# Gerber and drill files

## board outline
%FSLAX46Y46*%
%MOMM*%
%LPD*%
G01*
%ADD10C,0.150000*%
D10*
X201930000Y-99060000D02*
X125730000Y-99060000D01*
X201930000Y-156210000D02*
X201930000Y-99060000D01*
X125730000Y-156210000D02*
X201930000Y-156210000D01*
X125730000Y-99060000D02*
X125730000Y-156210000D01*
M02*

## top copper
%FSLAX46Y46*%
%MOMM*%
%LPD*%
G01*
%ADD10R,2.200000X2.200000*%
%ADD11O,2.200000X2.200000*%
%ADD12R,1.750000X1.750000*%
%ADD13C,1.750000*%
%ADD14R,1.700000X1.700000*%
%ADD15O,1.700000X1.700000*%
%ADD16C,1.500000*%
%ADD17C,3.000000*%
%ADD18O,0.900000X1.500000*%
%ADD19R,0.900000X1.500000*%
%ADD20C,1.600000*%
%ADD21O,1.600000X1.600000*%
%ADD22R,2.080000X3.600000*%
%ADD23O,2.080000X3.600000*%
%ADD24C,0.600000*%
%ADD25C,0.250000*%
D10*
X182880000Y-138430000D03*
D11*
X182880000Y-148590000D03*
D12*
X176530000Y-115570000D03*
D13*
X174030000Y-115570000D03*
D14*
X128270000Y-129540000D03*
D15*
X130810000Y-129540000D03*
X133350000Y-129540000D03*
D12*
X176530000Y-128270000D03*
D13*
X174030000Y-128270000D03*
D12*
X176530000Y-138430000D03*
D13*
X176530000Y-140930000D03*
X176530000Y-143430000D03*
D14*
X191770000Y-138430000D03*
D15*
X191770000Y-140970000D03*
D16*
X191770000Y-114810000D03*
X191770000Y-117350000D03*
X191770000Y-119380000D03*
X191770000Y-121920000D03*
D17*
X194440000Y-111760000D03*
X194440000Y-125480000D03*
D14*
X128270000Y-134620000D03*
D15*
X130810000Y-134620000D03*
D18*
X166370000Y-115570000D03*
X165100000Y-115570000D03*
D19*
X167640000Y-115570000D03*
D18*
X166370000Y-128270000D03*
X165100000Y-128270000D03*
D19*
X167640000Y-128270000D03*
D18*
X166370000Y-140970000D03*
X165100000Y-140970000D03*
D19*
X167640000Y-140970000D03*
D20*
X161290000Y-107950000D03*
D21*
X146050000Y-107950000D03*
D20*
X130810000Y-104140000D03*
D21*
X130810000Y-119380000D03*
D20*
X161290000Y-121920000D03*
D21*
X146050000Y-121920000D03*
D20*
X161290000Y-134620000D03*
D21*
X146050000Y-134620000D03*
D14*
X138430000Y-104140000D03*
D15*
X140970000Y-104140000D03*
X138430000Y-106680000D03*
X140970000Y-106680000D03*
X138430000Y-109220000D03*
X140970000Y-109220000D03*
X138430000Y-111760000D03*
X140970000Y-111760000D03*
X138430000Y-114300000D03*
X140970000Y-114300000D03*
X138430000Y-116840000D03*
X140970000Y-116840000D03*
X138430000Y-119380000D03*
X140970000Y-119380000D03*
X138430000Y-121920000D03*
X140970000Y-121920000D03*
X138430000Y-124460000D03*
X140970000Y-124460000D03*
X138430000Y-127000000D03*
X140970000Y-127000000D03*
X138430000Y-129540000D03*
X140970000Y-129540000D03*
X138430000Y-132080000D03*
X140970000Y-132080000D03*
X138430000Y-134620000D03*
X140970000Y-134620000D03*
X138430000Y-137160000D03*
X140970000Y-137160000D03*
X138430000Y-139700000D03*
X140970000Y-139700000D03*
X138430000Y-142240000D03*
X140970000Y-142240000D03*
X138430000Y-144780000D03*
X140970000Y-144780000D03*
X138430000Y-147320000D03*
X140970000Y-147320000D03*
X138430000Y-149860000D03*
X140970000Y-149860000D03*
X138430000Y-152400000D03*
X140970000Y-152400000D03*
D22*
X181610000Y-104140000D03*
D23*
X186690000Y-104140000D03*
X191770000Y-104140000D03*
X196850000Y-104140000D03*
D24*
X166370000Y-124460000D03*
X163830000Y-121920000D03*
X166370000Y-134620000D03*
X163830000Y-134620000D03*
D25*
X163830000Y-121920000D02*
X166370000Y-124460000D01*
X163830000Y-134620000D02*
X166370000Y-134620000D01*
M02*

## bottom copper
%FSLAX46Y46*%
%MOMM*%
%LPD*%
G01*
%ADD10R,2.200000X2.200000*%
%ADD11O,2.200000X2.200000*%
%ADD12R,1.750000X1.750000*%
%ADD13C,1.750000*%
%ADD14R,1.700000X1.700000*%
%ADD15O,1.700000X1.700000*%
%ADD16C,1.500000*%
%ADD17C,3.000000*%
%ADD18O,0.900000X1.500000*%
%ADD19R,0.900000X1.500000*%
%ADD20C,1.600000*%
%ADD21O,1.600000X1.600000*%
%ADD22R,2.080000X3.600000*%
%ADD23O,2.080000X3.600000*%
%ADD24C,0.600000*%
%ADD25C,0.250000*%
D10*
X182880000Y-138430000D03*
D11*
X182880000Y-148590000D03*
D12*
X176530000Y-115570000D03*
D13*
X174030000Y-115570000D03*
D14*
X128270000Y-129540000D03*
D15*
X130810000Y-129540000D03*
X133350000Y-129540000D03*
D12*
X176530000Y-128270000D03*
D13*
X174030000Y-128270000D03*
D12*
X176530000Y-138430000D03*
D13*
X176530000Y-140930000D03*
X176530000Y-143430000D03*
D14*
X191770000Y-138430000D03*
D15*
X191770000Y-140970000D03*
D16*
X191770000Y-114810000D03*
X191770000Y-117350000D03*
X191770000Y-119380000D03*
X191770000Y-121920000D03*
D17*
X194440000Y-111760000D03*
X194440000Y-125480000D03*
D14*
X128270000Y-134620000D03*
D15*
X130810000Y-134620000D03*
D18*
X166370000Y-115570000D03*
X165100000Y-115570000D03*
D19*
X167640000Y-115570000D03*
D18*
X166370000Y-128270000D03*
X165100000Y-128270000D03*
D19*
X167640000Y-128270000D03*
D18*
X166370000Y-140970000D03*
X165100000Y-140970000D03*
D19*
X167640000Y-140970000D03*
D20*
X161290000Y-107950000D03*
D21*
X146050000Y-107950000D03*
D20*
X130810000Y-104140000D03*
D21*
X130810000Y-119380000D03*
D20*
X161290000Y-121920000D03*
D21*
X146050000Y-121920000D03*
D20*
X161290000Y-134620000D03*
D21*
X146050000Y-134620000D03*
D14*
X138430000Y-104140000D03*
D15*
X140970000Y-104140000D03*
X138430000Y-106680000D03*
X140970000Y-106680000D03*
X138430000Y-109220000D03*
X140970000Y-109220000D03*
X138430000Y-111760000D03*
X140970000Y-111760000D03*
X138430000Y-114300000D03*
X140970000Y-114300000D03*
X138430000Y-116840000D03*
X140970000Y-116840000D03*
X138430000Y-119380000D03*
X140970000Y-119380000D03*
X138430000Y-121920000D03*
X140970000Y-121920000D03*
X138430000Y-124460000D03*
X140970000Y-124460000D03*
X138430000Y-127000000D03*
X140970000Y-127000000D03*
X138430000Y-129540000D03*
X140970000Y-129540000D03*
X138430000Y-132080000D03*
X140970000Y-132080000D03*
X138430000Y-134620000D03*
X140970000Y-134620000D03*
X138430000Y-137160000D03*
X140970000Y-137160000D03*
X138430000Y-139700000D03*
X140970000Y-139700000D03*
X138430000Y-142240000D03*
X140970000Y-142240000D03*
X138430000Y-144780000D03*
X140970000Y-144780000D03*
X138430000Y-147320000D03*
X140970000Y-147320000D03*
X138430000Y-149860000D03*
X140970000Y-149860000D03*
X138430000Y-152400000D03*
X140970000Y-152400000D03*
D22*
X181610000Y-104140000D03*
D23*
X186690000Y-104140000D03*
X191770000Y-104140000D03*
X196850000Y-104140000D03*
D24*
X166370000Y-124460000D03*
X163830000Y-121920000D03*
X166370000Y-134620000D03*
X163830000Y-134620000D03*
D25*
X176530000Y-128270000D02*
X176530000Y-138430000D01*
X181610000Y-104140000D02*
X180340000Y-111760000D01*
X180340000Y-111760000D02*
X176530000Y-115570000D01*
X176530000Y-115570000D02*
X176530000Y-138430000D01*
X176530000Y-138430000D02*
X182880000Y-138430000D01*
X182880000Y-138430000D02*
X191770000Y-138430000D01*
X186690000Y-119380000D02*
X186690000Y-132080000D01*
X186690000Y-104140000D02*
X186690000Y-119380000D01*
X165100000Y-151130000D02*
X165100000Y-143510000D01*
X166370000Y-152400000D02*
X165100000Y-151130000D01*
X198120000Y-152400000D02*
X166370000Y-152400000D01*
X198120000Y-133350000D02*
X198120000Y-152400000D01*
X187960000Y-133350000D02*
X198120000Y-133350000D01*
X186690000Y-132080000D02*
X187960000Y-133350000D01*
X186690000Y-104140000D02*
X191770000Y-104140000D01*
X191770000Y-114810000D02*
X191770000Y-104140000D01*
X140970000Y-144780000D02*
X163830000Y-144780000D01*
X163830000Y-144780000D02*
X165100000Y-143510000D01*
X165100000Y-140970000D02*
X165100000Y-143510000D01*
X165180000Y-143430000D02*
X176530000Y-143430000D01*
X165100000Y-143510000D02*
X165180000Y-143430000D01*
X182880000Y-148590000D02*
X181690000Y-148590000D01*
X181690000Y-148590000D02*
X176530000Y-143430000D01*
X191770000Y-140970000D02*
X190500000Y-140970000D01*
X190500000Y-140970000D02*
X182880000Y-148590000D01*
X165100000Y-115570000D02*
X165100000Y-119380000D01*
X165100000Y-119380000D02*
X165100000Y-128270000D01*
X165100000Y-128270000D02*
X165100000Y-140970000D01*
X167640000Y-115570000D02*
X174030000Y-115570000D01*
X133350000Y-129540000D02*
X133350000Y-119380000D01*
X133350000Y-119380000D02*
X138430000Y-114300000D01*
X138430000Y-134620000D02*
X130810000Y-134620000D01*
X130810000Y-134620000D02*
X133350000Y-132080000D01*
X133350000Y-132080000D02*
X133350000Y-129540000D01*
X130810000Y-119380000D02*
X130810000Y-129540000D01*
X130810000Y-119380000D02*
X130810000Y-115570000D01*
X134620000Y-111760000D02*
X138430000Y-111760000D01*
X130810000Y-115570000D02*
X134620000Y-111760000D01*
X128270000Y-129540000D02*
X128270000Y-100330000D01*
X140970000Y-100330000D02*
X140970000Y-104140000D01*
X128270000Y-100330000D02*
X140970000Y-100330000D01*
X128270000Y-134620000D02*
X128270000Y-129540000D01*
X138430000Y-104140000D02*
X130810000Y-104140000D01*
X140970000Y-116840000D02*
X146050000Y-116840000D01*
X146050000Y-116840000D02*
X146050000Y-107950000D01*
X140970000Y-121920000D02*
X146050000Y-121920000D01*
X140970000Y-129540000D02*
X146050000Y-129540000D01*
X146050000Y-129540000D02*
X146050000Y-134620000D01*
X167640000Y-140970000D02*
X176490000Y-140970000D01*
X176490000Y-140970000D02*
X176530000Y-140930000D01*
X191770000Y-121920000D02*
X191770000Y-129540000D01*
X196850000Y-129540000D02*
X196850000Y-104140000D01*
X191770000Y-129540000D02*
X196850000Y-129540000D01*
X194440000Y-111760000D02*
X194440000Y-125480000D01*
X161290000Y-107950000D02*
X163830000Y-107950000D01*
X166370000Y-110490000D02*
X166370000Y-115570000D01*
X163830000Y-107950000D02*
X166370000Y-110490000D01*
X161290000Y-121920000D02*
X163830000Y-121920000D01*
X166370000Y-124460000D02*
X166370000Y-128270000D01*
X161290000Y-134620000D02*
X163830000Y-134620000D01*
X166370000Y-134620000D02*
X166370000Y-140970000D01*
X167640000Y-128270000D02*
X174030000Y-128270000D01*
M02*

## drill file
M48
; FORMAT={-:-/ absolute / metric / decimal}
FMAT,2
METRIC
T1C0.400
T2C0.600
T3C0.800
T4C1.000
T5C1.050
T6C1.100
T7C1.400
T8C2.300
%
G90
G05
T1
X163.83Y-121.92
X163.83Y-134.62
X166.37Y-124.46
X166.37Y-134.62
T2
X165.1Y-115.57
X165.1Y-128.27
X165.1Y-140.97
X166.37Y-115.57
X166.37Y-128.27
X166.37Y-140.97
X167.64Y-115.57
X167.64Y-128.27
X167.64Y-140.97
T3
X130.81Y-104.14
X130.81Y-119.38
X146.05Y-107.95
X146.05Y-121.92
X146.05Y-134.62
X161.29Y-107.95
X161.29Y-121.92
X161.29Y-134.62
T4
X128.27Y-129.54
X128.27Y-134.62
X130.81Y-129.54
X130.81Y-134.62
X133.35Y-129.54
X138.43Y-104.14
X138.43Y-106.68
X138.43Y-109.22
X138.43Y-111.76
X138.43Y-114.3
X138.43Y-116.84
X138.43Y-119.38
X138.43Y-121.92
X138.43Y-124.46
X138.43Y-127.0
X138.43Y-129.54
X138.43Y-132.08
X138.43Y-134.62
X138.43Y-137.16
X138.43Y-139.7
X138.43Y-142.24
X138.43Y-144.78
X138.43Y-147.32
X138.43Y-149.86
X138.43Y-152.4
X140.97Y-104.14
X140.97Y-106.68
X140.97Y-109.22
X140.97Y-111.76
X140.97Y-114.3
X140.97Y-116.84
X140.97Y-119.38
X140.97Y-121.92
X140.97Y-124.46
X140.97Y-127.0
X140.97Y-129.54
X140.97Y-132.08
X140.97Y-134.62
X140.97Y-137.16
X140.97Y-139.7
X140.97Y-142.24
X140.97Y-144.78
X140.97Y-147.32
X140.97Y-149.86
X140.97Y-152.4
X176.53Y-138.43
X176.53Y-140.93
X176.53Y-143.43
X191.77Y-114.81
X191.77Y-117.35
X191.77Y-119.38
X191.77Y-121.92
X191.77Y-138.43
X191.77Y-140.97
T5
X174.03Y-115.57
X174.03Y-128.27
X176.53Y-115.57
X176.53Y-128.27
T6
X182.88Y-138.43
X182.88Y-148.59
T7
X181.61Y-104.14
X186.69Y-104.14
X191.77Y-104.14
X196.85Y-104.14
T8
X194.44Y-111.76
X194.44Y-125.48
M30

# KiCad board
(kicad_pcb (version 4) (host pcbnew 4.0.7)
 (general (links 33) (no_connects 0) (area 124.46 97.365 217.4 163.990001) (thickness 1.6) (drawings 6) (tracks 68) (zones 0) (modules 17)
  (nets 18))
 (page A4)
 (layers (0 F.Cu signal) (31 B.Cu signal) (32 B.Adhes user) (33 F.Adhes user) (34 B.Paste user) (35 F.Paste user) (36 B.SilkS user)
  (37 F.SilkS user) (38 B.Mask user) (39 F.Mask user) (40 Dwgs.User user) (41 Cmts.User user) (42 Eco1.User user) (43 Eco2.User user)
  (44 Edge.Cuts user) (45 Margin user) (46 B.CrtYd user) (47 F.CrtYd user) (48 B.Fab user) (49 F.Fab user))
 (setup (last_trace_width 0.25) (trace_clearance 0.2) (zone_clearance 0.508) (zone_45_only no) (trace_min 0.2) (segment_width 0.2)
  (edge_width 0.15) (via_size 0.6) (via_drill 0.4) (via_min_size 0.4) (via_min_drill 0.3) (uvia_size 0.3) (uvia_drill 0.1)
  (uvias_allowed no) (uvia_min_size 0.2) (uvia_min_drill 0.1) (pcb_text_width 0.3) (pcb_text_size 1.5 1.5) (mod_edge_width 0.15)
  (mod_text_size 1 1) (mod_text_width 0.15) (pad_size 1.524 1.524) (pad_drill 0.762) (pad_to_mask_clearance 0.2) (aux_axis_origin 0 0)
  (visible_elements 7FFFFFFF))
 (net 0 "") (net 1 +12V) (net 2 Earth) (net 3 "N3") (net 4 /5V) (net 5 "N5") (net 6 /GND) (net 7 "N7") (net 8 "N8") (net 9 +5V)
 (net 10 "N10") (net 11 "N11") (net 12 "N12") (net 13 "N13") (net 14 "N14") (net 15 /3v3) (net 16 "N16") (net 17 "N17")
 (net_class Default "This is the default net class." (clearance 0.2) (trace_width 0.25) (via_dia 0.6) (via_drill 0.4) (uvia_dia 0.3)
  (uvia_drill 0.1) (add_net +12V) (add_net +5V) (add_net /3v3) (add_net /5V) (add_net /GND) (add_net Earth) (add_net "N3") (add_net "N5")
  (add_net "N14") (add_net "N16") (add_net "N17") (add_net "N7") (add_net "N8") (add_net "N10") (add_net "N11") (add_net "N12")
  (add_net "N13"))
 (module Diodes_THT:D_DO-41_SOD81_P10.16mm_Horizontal (layer F.Cu) (at 182.88 138.43 270)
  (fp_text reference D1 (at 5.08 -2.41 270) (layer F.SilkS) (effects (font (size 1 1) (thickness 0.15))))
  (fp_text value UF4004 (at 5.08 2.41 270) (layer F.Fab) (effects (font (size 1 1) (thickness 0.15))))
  (pad 1 thru_hole rect (at 0 0 270) (size 2.2 2.2) (drill 1.1) (layers *.Cu *.Mask) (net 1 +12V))
  (pad 2 thru_hole oval (at 10.16 0 270) (size 2.2 2.2) (drill 1.1) (layers *.Cu *.Mask) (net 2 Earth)))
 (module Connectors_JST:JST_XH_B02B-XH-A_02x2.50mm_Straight (layer F.Cu) (at 176.53 115.57 180)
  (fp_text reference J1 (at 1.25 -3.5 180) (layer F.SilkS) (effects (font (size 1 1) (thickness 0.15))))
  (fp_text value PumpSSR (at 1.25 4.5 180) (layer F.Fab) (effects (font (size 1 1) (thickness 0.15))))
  (pad 1 thru_hole rect (at 0 0 180) (size 1.75 1.75) (drill 1.05) (layers *.Cu *.Mask) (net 1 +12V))
  (pad 2 thru_hole circle (at 2.5 0 180) (size 1.75 1.75) (drill 1.05) (layers *.Cu *.Mask) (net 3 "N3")))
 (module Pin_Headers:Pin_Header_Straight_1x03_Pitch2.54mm (layer F.Cu) (at 128.27 129.54 90)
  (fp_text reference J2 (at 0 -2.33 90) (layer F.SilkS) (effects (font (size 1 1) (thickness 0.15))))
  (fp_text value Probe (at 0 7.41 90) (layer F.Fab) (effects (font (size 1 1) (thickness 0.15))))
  (pad 1 thru_hole rect (at 0 0 90) (size 1.7 1.7) (drill 1) (layers *.Cu *.Mask) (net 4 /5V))
  (pad 2 thru_hole oval (at 0 2.54 90) (size 1.7 1.7) (drill 1) (layers *.Cu *.Mask) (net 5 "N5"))
  (pad 3 thru_hole oval (at 0 5.08 90) (size 1.7 1.7) (drill 1) (layers *.Cu *.Mask) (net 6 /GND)))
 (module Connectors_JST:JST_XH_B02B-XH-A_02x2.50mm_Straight (layer F.Cu) (at 176.53 128.27 180)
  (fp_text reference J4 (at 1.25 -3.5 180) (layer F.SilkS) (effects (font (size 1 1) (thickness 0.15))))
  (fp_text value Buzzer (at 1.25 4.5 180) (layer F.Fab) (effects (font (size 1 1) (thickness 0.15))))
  (pad 1 thru_hole rect (at 0 0 180) (size 1.75 1.75) (drill 1.05) (layers *.Cu *.Mask) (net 1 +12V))
  (pad 2 thru_hole circle (at 2.5 0 180) (size 1.75 1.75) (drill 1.05) (layers *.Cu *.Mask) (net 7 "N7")))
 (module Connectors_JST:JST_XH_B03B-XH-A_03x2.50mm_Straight (layer F.Cu) (at 176.53 138.43 270)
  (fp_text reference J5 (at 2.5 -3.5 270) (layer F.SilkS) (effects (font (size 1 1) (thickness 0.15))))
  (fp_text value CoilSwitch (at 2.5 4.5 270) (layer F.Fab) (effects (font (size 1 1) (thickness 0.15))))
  (pad 1 thru_hole rect (at 0 0 270) (size 1.75 1.75) (drill 1) (layers *.Cu *.Mask) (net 1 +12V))
  (pad 2 thru_hole circle (at 2.5 0 270) (size 1.75 1.75) (drill 1) (layers *.Cu *.Mask) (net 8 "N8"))
  (pad 3 thru_hole circle (at 5 0 270) (size 1.75 1.75) (drill 1) (layers *.Cu *.Mask) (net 2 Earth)))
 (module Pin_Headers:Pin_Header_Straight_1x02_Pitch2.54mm (layer F.Cu) (at 191.77 138.43)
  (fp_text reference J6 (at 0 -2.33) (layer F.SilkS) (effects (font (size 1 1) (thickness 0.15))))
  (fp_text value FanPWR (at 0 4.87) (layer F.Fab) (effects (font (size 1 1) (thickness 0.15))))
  (pad 1 thru_hole rect (at 0 0) (size 1.7 1.7) (drill 1) (layers *.Cu *.Mask) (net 1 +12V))
  (pad 2 thru_hole oval (at 0 2.54) (size 1.7 1.7) (drill 1) (layers *.Cu *.Mask) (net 2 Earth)))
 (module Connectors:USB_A (layer F.Cu) (at 191.77 121.92 90)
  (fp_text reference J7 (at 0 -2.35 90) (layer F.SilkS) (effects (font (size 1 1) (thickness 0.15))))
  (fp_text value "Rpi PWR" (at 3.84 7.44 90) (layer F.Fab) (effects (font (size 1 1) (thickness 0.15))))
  (pad 4 thru_hole circle (at 7.11 0) (size 1.5 1.5) (drill 1) (layers *.Cu *.Mask) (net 2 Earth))
  (pad 3 thru_hole circle (at 4.57 0) (size 1.5 1.5) (drill 1) (layers *.Cu *.Mask))
  (pad 2 thru_hole circle (at 2.54 0) (size 1.5 1.5) (drill 1) (layers *.Cu *.Mask))
  (pad 1 thru_hole circle (at 0 0) (size 1.5 1.5) (drill 1) (layers *.Cu *.Mask) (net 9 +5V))
  (pad 5 thru_hole circle (at 10.16 2.67) (size 3 3) (drill 2.3) (layers *.Cu *.Mask) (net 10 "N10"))
  (pad 5 thru_hole circle (at -3.56 2.67) (size 3 3) (drill 2.3) (layers *.Cu *.Mask) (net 10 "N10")))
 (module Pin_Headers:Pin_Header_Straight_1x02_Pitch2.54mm (layer F.Cu) (at 128.27 134.62 90)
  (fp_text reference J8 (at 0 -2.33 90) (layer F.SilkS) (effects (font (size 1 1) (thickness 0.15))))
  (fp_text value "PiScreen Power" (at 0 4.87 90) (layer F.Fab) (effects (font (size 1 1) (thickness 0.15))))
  (pad 1 thru_hole rect (at 0 0 90) (size 1.7 1.7) (drill 1) (layers *.Cu *.Mask) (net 4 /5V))
  (pad 2 thru_hole oval (at 0 2.54 90) (size 1.7 1.7) (drill 1) (layers *.Cu *.Mask) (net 6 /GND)))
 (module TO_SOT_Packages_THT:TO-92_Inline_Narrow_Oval (layer F.Cu) (at 167.64 115.57 180)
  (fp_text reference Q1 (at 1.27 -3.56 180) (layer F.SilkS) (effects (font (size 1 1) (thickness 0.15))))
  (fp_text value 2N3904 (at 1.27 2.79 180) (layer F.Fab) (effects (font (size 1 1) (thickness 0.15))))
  (pad 2 thru_hole oval (at 1.27 0) (size 0.9 1.5) (drill 0.6) (layers *.Cu *.Mask) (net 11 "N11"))
  (pad 3 thru_hole oval (at 2.54 0) (size 0.9 1.5) (drill 0.6) (layers *.Cu *.Mask) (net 2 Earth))
  (pad 1 thru_hole rect (at 0 0) (size 0.9 1.5) (drill 0.6) (layers *.Cu *.Mask) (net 3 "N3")))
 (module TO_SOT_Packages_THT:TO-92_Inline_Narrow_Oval (layer F.Cu) (at 167.64 128.27 180)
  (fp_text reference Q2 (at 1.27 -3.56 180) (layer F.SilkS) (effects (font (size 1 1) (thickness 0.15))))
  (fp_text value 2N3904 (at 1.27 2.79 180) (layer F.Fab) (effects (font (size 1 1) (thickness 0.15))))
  (pad 2 thru_hole oval (at 1.27 0) (size 0.9 1.5) (drill 0.6) (layers *.Cu *.Mask) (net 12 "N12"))
  (pad 3 thru_hole oval (at 2.54 0) (size 0.9 1.5) (drill 0.6) (layers *.Cu *.Mask) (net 2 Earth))
  (pad 1 thru_hole rect (at 0 0) (size 0.9 1.5) (drill 0.6) (layers *.Cu *.Mask) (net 7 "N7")))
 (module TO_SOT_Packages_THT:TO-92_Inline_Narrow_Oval (layer F.Cu) (at 167.64 140.97 180)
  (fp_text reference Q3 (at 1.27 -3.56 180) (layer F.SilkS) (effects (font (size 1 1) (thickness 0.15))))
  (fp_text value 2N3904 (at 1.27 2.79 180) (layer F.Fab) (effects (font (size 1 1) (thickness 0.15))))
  (pad 2 thru_hole oval (at 1.27 0) (size 0.9 1.5) (drill 0.6) (layers *.Cu *.Mask) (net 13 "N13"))
  (pad 3 thru_hole oval (at 2.54 0) (size 0.9 1.5) (drill 0.6) (layers *.Cu *.Mask) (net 2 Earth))
  (pad 1 thru_hole rect (at 0 0) (size 0.9 1.5) (drill 0.6) (layers *.Cu *.Mask) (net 8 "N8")))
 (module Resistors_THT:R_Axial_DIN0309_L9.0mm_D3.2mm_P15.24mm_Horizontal (layer F.Cu) (at 161.29 107.95 180)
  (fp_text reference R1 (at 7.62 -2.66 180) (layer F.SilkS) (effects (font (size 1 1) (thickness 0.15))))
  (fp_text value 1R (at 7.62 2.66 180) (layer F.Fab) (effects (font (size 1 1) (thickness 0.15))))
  (pad 1 thru_hole circle (at 0 0 180) (size 1.6 1.6) (drill 0.8) (layers *.Cu *.Mask) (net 11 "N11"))
  (pad 2 thru_hole oval (at 15.24 0 180) (size 1.6 1.6) (drill 0.8) (layers *.Cu *.Mask) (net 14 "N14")))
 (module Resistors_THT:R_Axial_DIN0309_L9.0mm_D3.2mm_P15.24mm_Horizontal (layer F.Cu) (at 130.81 104.14 270)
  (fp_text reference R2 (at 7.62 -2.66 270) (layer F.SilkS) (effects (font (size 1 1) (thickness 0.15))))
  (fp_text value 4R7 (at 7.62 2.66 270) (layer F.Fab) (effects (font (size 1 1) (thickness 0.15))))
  (pad 1 thru_hole circle (at 0 0 270) (size 1.6 1.6) (drill 0.8) (layers *.Cu *.Mask) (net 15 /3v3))
  (pad 2 thru_hole oval (at 15.24 0 270) (size 1.6 1.6) (drill 0.8) (layers *.Cu *.Mask) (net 5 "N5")))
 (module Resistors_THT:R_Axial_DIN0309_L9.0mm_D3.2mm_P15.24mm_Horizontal (layer F.Cu) (at 161.29 121.92 180)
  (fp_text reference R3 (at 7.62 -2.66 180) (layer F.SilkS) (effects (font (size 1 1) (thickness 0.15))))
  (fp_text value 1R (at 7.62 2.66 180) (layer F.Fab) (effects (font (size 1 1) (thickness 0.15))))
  (pad 1 thru_hole circle (at 0 0 180) (size 1.6 1.6) (drill 0.8) (layers *.Cu *.Mask) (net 12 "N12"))
  (pad 2 thru_hole oval (at 15.24 0 180) (size 1.6 1.6) (drill 0.8) (layers *.Cu *.Mask) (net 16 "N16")))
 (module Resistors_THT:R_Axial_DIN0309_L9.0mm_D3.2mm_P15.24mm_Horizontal (layer F.Cu) (at 161.29 134.62 180)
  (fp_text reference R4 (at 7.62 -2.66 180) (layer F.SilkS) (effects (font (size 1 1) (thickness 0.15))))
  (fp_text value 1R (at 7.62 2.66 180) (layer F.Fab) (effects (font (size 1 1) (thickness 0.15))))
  (pad 1 thru_hole circle (at 0 0 180) (size 1.6 1.6) (drill 0.8) (layers *.Cu *.Mask) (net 13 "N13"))
  (pad 2 thru_hole oval (at 15.24 0 180) (size 1.6 1.6) (drill 0.8) (layers *.Cu *.Mask) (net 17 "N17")))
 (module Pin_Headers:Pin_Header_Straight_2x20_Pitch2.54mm (layer F.Cu) (at 138.43 104.14)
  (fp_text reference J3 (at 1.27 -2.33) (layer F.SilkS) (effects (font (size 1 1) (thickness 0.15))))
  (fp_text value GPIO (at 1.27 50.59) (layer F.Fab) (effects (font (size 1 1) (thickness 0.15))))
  (pad 1 thru_hole rect (at 0 0) (size 1.7 1.7) (drill 1) (layers *.Cu *.Mask) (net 15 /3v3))
  (pad 2 thru_hole oval (at 2.54 0) (size 1.7 1.7) (drill 1) (layers *.Cu *.Mask) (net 4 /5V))
  (pad 3 thru_hole oval (at 0 2.54) (size 1.7 1.7) (drill 1) (layers *.Cu *.Mask))
  (pad 4 thru_hole oval (at 2.54 2.54) (size 1.7 1.7) (drill 1) (layers *.Cu *.Mask))
  (pad 5 thru_hole oval (at 0 5.08) (size 1.7 1.7) (drill 1) (layers *.Cu *.Mask))
  (pad 6 thru_hole oval (at 2.54 5.08) (size 1.7 1.7) (drill 1) (layers *.Cu *.Mask))
  (pad 7 thru_hole oval (at 0 7.62) (size 1.7 1.7) (drill 1) (layers *.Cu *.Mask) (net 5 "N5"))
  (pad 8 thru_hole oval (at 2.54 7.62) (size 1.7 1.7) (drill 1) (layers *.Cu *.Mask))
  (pad 9 thru_hole oval (at 0 10.16) (size 1.7 1.7) (drill 1) (layers *.Cu *.Mask) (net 6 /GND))
  (pad 10 thru_hole oval (at 2.54 10.16) (size 1.7 1.7) (drill 1) (layers *.Cu *.Mask))
  (pad 11 thru_hole oval (at 0 12.7) (size 1.7 1.7) (drill 1) (layers *.Cu *.Mask))
  (pad 12 thru_hole oval (at 2.54 12.7) (size 1.7 1.7) (drill 1) (layers *.Cu *.Mask) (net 14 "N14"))
  (pad 13 thru_hole oval (at 0 15.24) (size 1.7 1.7) (drill 1) (layers *.Cu *.Mask))
  (pad 14 thru_hole oval (at 2.54 15.24) (size 1.7 1.7) (drill 1) (layers *.Cu *.Mask))
  (pad 15 thru_hole oval (at 0 17.78) (size 1.7 1.7) (drill 1) (layers *.Cu *.Mask))
  (pad 16 thru_hole oval (at 2.54 17.78) (size 1.7 1.7) (drill 1) (layers *.Cu *.Mask) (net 16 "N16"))
  (pad 17 thru_hole oval (at 0 20.32) (size 1.7 1.7) (drill 1) (layers *.Cu *.Mask))
  (pad 18 thru_hole oval (at 2.54 20.32) (size 1.7 1.7) (drill 1) (layers *.Cu *.Mask))
  (pad 19 thru_hole oval (at 0 22.86) (size 1.7 1.7) (drill 1) (layers *.Cu *.Mask))
  (pad 20 thru_hole oval (at 2.54 22.86) (size 1.7 1.7) (drill 1) (layers *.Cu *.Mask))
  (pad 21 thru_hole oval (at 0 25.4) (size 1.7 1.7) (drill 1) (layers *.Cu *.Mask))
  (pad 22 thru_hole oval (at 2.54 25.4) (size 1.7 1.7) (drill 1) (layers *.Cu *.Mask) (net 17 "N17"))
  (pad 23 thru_hole oval (at 0 27.94) (size 1.7 1.7) (drill 1) (layers *.Cu *.Mask))
  (pad 24 thru_hole oval (at 2.54 27.94) (size 1.7 1.7) (drill 1) (layers *.Cu *.Mask))
  (pad 25 thru_hole oval (at 0 30.48) (size 1.7 1.7) (drill 1) (layers *.Cu *.Mask) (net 6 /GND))
  (pad 26 thru_hole oval (at 2.54 30.48) (size 1.7 1.7) (drill 1) (layers *.Cu *.Mask))
  (pad 27 thru_hole oval (at 0 33.02) (size 1.7 1.7) (drill 1) (layers *.Cu *.Mask))
  (pad 28 thru_hole oval (at 2.54 33.02) (size 1.7 1.7) (drill 1) (layers *.Cu *.Mask))
  (pad 29 thru_hole oval (at 0 35.56) (size 1.7 1.7) (drill 1) (layers *.Cu *.Mask))
  (pad 30 thru_hole oval (at 2.54 35.56) (size 1.7 1.7) (drill 1) (layers *.Cu *.Mask))
  (pad 31 thru_hole oval (at 0 38.1) (size 1.7 1.7) (drill 1) (layers *.Cu *.Mask))
  (pad 32 thru_hole oval (at 2.54 38.1) (size 1.7 1.7) (drill 1) (layers *.Cu *.Mask))
  (pad 33 thru_hole oval (at 0 40.64) (size 1.7 1.7) (drill 1) (layers *.Cu *.Mask))
  (pad 34 thru_hole oval (at 2.54 40.64) (size 1.7 1.7) (drill 1) (layers *.Cu *.Mask) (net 2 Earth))
  (pad 35 thru_hole oval (at 0 43.18) (size 1.7 1.7) (drill 1) (layers *.Cu *.Mask))
  (pad 36 thru_hole oval (at 2.54 43.18) (size 1.7 1.7) (drill 1) (layers *.Cu *.Mask))
  (pad 37 thru_hole oval (at 0 45.72) (size 1.7 1.7) (drill 1) (layers *.Cu *.Mask))
  (pad 38 thru_hole oval (at 2.54 45.72) (size 1.7 1.7) (drill 1) (layers *.Cu *.Mask))
  (pad 39 thru_hole oval (at 0 48.26) (size 1.7 1.7) (drill 1) (layers *.Cu *.Mask))
  (pad 40 thru_hole oval (at 2.54 48.26) (size 1.7 1.7) (drill 1) (layers *.Cu *.Mask)))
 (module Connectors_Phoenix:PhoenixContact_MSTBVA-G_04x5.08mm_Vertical (layer F.Cu) (at 181.61 104.14)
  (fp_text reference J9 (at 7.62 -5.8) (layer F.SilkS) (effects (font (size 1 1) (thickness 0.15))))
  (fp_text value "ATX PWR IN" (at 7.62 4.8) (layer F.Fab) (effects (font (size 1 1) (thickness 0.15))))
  (pad 1 thru_hole rect (at 0 0) (size 2.08 3.6) (drill 1.4) (layers *.Cu *.Mask) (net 1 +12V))
  (pad 2 thru_hole oval (at 5.08 0) (size 2.08 3.6) (drill 1.4) (layers *.Cu *.Mask) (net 2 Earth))
  (pad 3 thru_hole oval (at 10.16 0) (size 2.08 3.6) (drill 1.4) (layers *.Cu *.Mask) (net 2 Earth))
  (pad 4 thru_hole oval (at 15.24 0) (size 2.08 3.6) (drill 1.4) (layers *.Cu *.Mask) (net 9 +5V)))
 (gr_line (start 201.93 99.06) (end 125.73 99.06) (angle 90) (layer Edge.Cuts) (width 0.15))
 (gr_line (start 201.93 156.21) (end 201.93 99.06) (angle 90) (layer Edge.Cuts) (width 0.15))
 (gr_line (start 125.73 156.21) (end 201.93 156.21) (angle 90) (layer Edge.Cuts) (width 0.15))
 (gr_line (start 125.73 99.06) (end 125.73 156.21) (angle 90) (layer Edge.Cuts) (width 0.15))
 (segment (start 176.53 128.27) (end 176.53 138.43) (width 0.25) (layer B.Cu) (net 1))
 (segment (start 181.61 104.14) (end 180.34 111.76) (width 0.25) (layer B.Cu) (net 1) (status 10))
 (segment (start 180.34 111.76) (end 176.53 115.57) (width 0.25) (layer B.Cu) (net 1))
 (segment (start 176.53 115.57) (end 176.53 138.43) (width 0.25) (layer B.Cu) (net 1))
 (segment (start 176.53 138.43) (end 182.88 138.43) (width 0.25) (layer B.Cu) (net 1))
 (segment (start 182.88 138.43) (end 191.77 138.43) (width 0.25) (layer B.Cu) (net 1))
 (segment (start 186.69 119.38) (end 186.69 132.08) (width 0.25) (layer B.Cu) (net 2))
 (segment (start 186.69 104.14) (end 186.69 119.38) (width 0.25) (layer B.Cu) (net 2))
 (segment (start 165.1 151.13) (end 165.1 143.51) (width 0.25) (layer B.Cu) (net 2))
 (segment (start 166.37 152.4) (end 165.1 151.13) (width 0.25) (layer B.Cu) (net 2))
 (segment (start 198.12 152.4) (end 166.37 152.4) (width 0.25) (layer B.Cu) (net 2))
 (segment (start 198.12 133.35) (end 198.12 152.4) (width 0.25) (layer B.Cu) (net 2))
 (segment (start 187.96 133.35) (end 198.12 133.35) (width 0.25) (layer B.Cu) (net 2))
 (segment (start 186.69 132.08) (end 187.96 133.35) (width 0.25) (layer B.Cu) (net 2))
 (segment (start 186.69 104.14) (end 191.77 104.14) (width 0.25) (layer B.Cu) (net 2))
 (segment (start 191.77 114.81) (end 191.77 104.14) (width 0.25) (layer B.Cu) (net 2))
 (segment (start 140.97 144.78) (end 163.83 144.78) (width 0.25) (layer B.Cu) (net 2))
 (segment (start 163.83 144.78) (end 165.1 143.51) (width 0.25) (layer B.Cu) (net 2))
 (segment (start 165.1 140.97) (end 165.1 143.51) (width 0.25) (layer B.Cu) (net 2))
 (segment (start 165.18 143.43) (end 176.53 143.43) (width 0.25) (layer B.Cu) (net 2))
 (segment (start 165.1 143.51) (end 165.18 143.43) (width 0.25) (layer B.Cu) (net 2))
 (segment (start 182.88 148.59) (end 181.69 148.59) (width 0.25) (layer B.Cu) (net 2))
 (segment (start 181.69 148.59) (end 176.53 143.43) (width 0.25) (layer B.Cu) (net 2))
 (segment (start 191.77 140.97) (end 190.5 140.97) (width 0.25) (layer B.Cu) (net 2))
 (segment (start 190.5 140.97) (end 182.88 148.59) (width 0.25) (layer B.Cu) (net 2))
 (segment (start 165.1 115.57) (end 165.1 119.38) (width 0.25) (layer B.Cu) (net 2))
 (segment (start 165.1 119.38) (end 165.1 128.27) (width 0.25) (layer B.Cu) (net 2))
 (segment (start 165.1 128.27) (end 165.1 140.97) (width 0.25) (layer B.Cu) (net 2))
 (segment (start 167.64 115.57) (end 174.03 115.57) (width 0.25) (layer B.Cu) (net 3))
 (segment (start 133.35 129.54) (end 133.35 119.38) (width 0.25) (layer B.Cu) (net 6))
 (segment (start 133.35 119.38) (end 138.43 114.3) (width 0.25) (layer B.Cu) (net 6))
 (segment (start 138.43 134.62) (end 130.81 134.62) (width 0.25) (layer B.Cu) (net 6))
 (segment (start 130.81 134.62) (end 133.35 132.08) (width 0.25) (layer B.Cu) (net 6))
 (segment (start 133.35 132.08) (end 133.35 129.54) (width 0.25) (layer B.Cu) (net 6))
 (segment (start 130.81 119.38) (end 130.81 129.54) (width 0.25) (layer B.Cu) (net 5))
 (segment (start 130.81 119.38) (end 130.81 115.57) (width 0.25) (layer B.Cu) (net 5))
 (segment (start 134.62 111.76) (end 138.43 111.76) (width 0.25) (layer B.Cu) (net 5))
 (segment (start 130.81 115.57) (end 134.62 111.76) (width 0.25) (layer B.Cu) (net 5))
 (segment (start 128.27 129.54) (end 128.27 100.33) (width 0.25) (layer B.Cu) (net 4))
 (segment (start 140.97 100.33) (end 140.97 104.14) (width 0.25) (layer B.Cu) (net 4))
 (segment (start 128.27 100.33) (end 140.97 100.33) (width 0.25) (layer B.Cu) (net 4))
 (segment (start 128.27 134.62) (end 128.27 129.54) (width 0.25) (layer B.Cu) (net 4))
 (segment (start 138.43 104.14) (end 130.81 104.14) (width 0.25) (layer B.Cu) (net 15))
 (segment (start 140.97 116.84) (end 146.05 116.84) (width 0.25) (layer B.Cu) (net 14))
 (segment (start 146.05 116.84) (end 146.05 107.95) (width 0.25) (layer B.Cu) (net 14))
 (segment (start 140.97 121.92) (end 146.05 121.92) (width 0.25) (layer B.Cu) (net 16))
 (segment (start 140.97 129.54) (end 146.05 129.54) (width 0.25) (layer B.Cu) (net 17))
 (segment (start 146.05 129.54) (end 146.05 134.62) (width 0.25) (layer B.Cu) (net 17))
 (segment (start 167.64 140.97) (end 176.49 140.97) (width 0.25) (layer B.Cu) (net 8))
 (segment (start 176.49 140.97) (end 176.53 140.93) (width 0.25) (layer B.Cu) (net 8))
 (segment (start 191.77 121.92) (end 191.77 129.54) (width 0.25) (layer B.Cu) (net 9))
 (segment (start 196.85 129.54) (end 196.85 104.14) (width 0.25) (layer B.Cu) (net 9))
 (segment (start 191.77 129.54) (end 196.85 129.54) (width 0.25) (layer B.Cu) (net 9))
 (segment (start 194.44 111.76) (end 194.44 125.48) (width 0.25) (layer B.Cu) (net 10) (status 30))
 (segment (start 161.29 107.95) (end 163.83 107.95) (width 0.25) (layer B.Cu) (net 11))
 (segment (start 166.37 110.49) (end 166.37 115.57) (width 0.25) (layer B.Cu) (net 11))
 (segment (start 163.83 107.95) (end 166.37 110.49) (width 0.25) (layer B.Cu) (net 11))
 (segment (start 161.29 121.92) (end 163.83 121.92) (width 0.25) (layer B.Cu) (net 12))
 (segment (start 166.37 124.46) (end 166.37 128.27) (width 0.25) (layer B.Cu) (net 12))
 (via (at 166.37 124.46) (size 0.6) (drill 0.4) (layers F.Cu B.Cu) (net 12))
 (segment (start 163.83 121.92) (end 166.37 124.46) (width 0.25) (layer F.Cu) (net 12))
 (via (at 163.83 121.92) (size 0.6) (drill 0.4) (layers F.Cu B.Cu) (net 12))
 (segment (start 161.29 134.62) (end 163.83 134.62) (width 0.25) (layer B.Cu) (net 13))
 (segment (start 166.37 134.62) (end 166.37 140.97) (width 0.25) (layer B.Cu) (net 13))
 (via (at 166.37 134.62) (size 0.6) (drill 0.4) (layers F.Cu B.Cu) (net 13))
 (segment (start 163.83 134.62) (end 166.37 134.62) (width 0.25) (layer F.Cu) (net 13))
 (via (at 163.83 134.62) (size 0.6) (drill 0.4) (layers F.Cu B.Cu) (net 13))
 (segment (start 167.64 128.27) (end 174.03 128.27) (width 0.25) (layer B.Cu) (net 7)))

